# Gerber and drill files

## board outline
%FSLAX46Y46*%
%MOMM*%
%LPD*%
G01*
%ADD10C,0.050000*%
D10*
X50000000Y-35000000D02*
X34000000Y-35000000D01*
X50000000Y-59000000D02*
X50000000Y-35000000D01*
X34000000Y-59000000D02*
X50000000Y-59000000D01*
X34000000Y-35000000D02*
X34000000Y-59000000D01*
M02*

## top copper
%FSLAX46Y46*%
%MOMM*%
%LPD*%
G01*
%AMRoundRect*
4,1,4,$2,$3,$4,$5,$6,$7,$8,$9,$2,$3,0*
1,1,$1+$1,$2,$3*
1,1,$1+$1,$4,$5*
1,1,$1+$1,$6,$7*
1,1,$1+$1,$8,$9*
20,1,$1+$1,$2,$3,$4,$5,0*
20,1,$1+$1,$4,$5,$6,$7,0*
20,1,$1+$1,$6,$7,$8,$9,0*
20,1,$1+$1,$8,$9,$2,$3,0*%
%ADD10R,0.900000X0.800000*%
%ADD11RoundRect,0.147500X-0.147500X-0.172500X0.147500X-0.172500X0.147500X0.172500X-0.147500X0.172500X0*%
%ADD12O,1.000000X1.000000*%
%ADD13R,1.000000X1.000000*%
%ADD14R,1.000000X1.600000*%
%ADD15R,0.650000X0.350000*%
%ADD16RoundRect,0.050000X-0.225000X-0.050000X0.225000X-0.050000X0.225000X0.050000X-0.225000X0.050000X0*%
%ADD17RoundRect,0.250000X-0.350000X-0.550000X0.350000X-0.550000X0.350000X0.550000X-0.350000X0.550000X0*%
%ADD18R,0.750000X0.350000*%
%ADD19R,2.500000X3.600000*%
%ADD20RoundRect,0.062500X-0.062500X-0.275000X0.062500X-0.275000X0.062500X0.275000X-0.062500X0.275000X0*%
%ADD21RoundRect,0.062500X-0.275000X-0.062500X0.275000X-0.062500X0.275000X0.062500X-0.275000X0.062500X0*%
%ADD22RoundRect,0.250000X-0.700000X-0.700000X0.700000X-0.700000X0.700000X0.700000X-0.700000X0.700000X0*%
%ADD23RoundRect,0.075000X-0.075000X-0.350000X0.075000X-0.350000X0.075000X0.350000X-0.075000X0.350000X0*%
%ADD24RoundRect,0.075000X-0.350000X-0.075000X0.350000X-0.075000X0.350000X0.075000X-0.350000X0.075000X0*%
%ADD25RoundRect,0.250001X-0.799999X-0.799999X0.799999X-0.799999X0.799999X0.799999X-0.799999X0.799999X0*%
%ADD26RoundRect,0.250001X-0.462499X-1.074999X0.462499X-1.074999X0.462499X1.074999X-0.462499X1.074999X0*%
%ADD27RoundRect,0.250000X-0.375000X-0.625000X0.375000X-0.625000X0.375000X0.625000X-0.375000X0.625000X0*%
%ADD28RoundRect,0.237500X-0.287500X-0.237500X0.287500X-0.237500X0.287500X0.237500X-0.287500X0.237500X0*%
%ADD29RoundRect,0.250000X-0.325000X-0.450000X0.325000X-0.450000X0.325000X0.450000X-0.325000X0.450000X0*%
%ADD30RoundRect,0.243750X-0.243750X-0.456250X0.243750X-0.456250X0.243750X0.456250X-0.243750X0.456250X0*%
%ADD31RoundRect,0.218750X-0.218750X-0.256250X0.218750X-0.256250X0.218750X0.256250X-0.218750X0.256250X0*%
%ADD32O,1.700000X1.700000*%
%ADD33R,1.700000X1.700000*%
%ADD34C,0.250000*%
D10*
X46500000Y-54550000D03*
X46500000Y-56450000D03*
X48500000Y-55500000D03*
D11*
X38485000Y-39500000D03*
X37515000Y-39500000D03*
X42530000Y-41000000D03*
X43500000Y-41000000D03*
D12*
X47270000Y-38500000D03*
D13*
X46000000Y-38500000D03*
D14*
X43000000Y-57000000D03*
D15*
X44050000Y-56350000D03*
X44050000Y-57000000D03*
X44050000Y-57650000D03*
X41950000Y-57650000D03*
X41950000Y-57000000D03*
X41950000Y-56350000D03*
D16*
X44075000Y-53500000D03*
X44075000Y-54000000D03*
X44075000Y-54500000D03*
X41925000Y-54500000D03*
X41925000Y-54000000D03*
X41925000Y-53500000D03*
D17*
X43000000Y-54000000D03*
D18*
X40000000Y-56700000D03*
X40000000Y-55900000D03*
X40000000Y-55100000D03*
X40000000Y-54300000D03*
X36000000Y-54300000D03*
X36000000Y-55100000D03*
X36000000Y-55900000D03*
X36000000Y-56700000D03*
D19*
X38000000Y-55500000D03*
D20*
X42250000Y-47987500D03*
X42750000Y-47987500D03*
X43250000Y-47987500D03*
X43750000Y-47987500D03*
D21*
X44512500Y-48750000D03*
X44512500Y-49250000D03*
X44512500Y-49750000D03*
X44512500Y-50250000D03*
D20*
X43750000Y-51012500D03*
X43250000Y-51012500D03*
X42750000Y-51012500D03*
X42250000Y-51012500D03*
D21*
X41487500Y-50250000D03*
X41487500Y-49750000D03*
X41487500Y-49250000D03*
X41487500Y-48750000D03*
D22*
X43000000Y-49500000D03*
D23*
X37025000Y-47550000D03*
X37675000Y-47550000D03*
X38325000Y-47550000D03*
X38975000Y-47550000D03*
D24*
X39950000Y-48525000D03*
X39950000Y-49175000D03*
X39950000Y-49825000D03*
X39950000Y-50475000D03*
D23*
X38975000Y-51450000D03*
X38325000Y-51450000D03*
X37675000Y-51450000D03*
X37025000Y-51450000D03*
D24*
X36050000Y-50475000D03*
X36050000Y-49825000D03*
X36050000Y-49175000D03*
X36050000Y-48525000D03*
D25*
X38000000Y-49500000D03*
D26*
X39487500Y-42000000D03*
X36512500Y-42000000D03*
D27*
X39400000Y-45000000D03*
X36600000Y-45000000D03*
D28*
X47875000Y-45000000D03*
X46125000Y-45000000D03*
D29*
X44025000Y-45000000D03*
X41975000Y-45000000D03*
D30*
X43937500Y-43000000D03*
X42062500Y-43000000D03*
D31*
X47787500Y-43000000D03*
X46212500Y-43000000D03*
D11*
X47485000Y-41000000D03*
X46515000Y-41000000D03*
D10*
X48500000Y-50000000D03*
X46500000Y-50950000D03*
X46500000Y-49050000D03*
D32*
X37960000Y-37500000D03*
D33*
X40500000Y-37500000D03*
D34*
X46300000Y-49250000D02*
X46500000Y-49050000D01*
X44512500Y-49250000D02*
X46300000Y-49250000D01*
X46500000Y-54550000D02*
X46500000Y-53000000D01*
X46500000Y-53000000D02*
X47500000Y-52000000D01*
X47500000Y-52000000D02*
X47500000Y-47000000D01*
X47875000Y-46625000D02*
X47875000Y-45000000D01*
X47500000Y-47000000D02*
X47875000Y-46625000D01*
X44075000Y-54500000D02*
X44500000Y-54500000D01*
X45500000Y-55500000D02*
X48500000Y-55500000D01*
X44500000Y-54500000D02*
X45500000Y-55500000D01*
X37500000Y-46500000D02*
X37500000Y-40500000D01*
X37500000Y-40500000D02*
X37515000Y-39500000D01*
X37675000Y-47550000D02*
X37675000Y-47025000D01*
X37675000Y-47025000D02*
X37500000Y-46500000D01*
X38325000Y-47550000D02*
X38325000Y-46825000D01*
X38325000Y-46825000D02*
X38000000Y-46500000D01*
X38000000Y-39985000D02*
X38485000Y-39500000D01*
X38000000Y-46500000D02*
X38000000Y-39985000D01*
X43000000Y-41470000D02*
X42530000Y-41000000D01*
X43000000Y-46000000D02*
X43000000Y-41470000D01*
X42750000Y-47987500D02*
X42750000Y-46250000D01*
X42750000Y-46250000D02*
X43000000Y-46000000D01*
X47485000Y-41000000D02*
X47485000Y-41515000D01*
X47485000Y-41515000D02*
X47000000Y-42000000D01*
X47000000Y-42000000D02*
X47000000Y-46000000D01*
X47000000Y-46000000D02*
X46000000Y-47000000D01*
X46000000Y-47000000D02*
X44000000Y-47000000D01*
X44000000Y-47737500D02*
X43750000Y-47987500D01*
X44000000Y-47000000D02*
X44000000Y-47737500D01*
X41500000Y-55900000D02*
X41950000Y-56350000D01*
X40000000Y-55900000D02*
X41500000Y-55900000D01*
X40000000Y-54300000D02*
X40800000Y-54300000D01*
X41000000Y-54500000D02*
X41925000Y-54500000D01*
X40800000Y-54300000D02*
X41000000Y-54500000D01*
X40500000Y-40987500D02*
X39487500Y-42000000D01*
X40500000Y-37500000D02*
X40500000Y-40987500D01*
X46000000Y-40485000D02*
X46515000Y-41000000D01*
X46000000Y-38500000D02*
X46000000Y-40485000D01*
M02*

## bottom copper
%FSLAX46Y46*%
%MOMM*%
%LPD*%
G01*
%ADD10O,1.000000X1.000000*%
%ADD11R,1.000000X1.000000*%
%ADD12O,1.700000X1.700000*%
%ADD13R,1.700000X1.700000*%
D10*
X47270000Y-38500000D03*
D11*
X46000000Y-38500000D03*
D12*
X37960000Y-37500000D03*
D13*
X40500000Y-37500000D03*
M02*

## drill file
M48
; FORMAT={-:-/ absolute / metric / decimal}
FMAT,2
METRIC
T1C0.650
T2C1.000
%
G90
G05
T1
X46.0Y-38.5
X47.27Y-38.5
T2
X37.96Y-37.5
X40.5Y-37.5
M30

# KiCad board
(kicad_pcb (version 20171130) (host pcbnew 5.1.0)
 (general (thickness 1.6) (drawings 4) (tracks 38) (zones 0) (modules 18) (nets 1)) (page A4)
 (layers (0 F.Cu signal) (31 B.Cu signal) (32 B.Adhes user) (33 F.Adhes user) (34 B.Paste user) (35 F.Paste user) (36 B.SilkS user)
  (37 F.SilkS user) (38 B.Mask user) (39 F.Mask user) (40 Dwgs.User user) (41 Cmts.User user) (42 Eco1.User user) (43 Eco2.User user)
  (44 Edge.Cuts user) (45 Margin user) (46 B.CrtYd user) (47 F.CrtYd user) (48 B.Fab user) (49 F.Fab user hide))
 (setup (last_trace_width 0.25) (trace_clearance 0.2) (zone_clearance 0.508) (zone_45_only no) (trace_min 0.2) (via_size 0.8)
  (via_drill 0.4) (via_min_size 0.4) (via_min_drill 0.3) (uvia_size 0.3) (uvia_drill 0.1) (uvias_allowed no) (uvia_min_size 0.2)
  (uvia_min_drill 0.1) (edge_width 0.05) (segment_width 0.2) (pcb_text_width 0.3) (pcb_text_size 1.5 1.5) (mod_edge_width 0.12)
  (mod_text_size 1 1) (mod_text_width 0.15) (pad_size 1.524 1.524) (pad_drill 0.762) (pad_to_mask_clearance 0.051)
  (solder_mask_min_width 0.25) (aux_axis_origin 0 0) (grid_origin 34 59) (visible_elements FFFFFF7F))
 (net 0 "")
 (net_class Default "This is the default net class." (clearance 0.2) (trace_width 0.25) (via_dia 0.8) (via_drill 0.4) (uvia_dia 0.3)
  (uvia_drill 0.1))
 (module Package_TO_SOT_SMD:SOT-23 (layer F.Cu) (at 47.5 55.5)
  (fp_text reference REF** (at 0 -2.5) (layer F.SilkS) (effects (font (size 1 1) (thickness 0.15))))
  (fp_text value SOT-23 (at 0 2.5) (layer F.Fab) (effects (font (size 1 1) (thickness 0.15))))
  (pad 1 smd rect (at -1 -0.95) (size 0.9 0.8) (layers F.Cu F.Paste F.Mask))
  (pad 2 smd rect (at -1 0.95) (size 0.9 0.8) (layers F.Cu F.Paste F.Mask))
  (pad 3 smd rect (at 1 0) (size 0.9 0.8) (layers F.Cu F.Paste F.Mask)))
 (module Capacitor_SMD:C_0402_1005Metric (layer F.Cu) (at 38 39.5)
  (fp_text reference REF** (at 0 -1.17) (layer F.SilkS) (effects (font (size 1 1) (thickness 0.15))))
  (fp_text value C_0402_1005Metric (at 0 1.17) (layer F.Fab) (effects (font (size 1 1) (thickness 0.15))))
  (pad 2 smd roundrect (at 0.485 0) (size 0.59 0.64) (layers F.Cu F.Paste F.Mask) (roundrect_rratio 0.25))
  (pad 1 smd roundrect (at -0.485 0) (size 0.59 0.64) (layers F.Cu F.Paste F.Mask) (roundrect_rratio 0.25)))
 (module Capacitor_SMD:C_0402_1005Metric (layer F.Cu) (at 43.015 41)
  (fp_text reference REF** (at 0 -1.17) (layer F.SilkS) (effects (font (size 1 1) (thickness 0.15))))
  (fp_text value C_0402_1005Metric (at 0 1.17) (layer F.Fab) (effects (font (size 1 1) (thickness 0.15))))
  (pad 1 smd roundrect (at -0.485 0) (size 0.59 0.64) (layers F.Cu F.Paste F.Mask) (roundrect_rratio 0.25))
  (pad 2 smd roundrect (at 0.485 0) (size 0.59 0.64) (layers F.Cu F.Paste F.Mask) (roundrect_rratio 0.25)))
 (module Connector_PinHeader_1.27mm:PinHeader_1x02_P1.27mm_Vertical (layer F.Cu) (at 46 38.5 90)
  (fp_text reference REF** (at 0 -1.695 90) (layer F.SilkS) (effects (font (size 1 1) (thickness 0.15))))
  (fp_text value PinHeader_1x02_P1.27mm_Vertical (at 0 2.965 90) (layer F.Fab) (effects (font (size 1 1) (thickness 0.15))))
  (pad 2 thru_hole oval (at 0 1.27 90) (size 1 1) (drill 0.65) (layers *.Cu *.Mask))
  (pad 1 thru_hole rect (at 0 0 90) (size 1 1) (drill 0.65) (layers *.Cu *.Mask)))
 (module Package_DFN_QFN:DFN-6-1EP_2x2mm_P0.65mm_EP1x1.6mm (layer F.Cu) (at 43 57)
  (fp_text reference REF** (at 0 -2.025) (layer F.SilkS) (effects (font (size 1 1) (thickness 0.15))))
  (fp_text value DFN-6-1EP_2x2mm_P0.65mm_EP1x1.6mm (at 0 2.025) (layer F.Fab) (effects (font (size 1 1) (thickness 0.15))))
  (pad "" smd rect (at 0 0.4) (size 0.82 0.63) (layers F.Paste))
  (pad "" smd rect (at 0 -0.4) (size 0.82 0.63) (layers F.Paste)) (pad 7 smd rect (at 0 0) (size 1 1.6) (layers F.Cu F.Mask))
  (pad 6 smd rect (at 1.05 -0.65) (size 0.65 0.35) (layers F.Cu F.Paste F.Mask))
  (pad 5 smd rect (at 1.05 0) (size 0.65 0.35) (layers F.Cu F.Paste F.Mask))
  (pad 4 smd rect (at 1.05 0.65) (size 0.65 0.35) (layers F.Cu F.Paste F.Mask))
  (pad 3 smd rect (at -1.05 0.65) (size 0.65 0.35) (layers F.Cu F.Paste F.Mask))
  (pad 2 smd rect (at -1.05 0) (size 0.65 0.35) (layers F.Cu F.Paste F.Mask))
  (pad 1 smd rect (at -1.05 -0.65) (size 0.65 0.35) (layers F.Cu F.Paste F.Mask)))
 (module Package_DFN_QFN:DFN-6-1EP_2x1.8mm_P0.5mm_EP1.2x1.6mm (layer F.Cu) (at 43 54)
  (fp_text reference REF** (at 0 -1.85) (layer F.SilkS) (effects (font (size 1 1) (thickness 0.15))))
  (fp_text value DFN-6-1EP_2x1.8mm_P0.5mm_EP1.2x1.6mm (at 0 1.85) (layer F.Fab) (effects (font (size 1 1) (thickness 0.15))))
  (pad 6 smd roundrect (at 1.075 -0.5) (size 0.55 0.2) (layers F.Cu F.Paste F.Mask) (roundrect_rratio 0.25))
  (pad 5 smd roundrect (at 1.075 0) (size 0.55 0.2) (layers F.Cu F.Paste F.Mask) (roundrect_rratio 0.25))
  (pad 4 smd roundrect (at 1.075 0.5) (size 0.55 0.2) (layers F.Cu F.Paste F.Mask) (roundrect_rratio 0.25))
  (pad 3 smd roundrect (at -1.075 0.5) (size 0.55 0.2) (layers F.Cu F.Paste F.Mask) (roundrect_rratio 0.25))
  (pad 2 smd roundrect (at -1.075 0) (size 0.55 0.2) (layers F.Cu F.Paste F.Mask) (roundrect_rratio 0.25))
  (pad 1 smd roundrect (at -1.075 -0.5) (size 0.55 0.2) (layers F.Cu F.Paste F.Mask) (roundrect_rratio 0.25))
  (pad "" smd roundrect (at 0.3 0.4) (size 0.48 0.64) (layers F.Paste) (roundrect_rratio 0.25))
  (pad "" smd roundrect (at 0.3 -0.4) (size 0.48 0.64) (layers F.Paste) (roundrect_rratio 0.25))
  (pad "" smd roundrect (at -0.3 0.4) (size 0.48 0.64) (layers F.Paste) (roundrect_rratio 0.25))
  (pad "" smd roundrect (at -0.3 -0.4) (size 0.48 0.64) (layers F.Paste) (roundrect_rratio 0.25))
  (pad 7 smd roundrect (at 0 0) (size 1.2 1.6) (layers F.Cu F.Mask) (roundrect_rratio 0.208333)))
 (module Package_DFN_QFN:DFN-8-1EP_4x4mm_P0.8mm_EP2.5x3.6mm (layer F.Cu) (at 38 55.5 180)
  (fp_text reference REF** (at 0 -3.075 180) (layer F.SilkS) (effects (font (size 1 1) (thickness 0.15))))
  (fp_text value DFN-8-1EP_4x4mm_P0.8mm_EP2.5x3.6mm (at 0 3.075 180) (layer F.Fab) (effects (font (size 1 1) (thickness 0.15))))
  (pad 1 smd rect (at -2 -1.2 180) (size 0.75 0.35) (layers F.Cu F.Paste F.Mask))
  (pad 2 smd rect (at -2 -0.4 180) (size 0.75 0.35) (layers F.Cu F.Paste F.Mask))
  (pad 3 smd rect (at -2 0.4 180) (size 0.75 0.35) (layers F.Cu F.Paste F.Mask))
  (pad 4 smd rect (at -2 1.2 180) (size 0.75 0.35) (layers F.Cu F.Paste F.Mask))
  (pad 5 smd rect (at 2 1.2 180) (size 0.75 0.35) (layers F.Cu F.Paste F.Mask))
  (pad 6 smd rect (at 2 0.4 180) (size 0.75 0.35) (layers F.Cu F.Paste F.Mask))
  (pad 7 smd rect (at 2 -0.4 180) (size 0.75 0.35) (layers F.Cu F.Paste F.Mask))
  (pad 8 smd rect (at 2 -1.2 180) (size 0.75 0.35) (layers F.Cu F.Paste F.Mask))
  (pad "" smd rect (at -0.625 -1.2 180) (size 1 1) (layers F.Paste))
  (pad 9 smd rect (at 0 0 180) (size 2.5 3.6) (layers F.Cu F.Mask))
  (pad "" smd rect (at 0.625 -1.2 180) (size 1 1) (layers F.Paste))
  (pad "" smd rect (at 0.625 0 180) (size 1 1) (layers F.Paste))
  (pad "" smd rect (at -0.625 0 180) (size 1 1) (layers F.Paste))
  (pad "" smd rect (at 0.625 1.2 180) (size 1 1) (layers F.Paste))
  (pad "" smd rect (at -0.625 1.2 180) (size 1 1) (layers F.Paste)))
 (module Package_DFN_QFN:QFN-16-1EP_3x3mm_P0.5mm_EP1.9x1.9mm (layer F.Cu) (at 43 49.5)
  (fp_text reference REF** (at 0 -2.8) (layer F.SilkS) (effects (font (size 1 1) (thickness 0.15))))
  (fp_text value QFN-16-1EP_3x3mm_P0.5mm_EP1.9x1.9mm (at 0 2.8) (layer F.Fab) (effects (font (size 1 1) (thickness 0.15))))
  (pad 16 smd roundrect (at -0.75 -1.5125) (size 0.25 0.675) (layers F.Cu F.Paste F.Mask) (roundrect_rratio 0.25))
  (pad 15 smd roundrect (at -0.25 -1.5125) (size 0.25 0.675) (layers F.Cu F.Paste F.Mask) (roundrect_rratio 0.25))
  (pad 14 smd roundrect (at 0.25 -1.5125) (size 0.25 0.675) (layers F.Cu F.Paste F.Mask) (roundrect_rratio 0.25))
  (pad 13 smd roundrect (at 0.75 -1.5125) (size 0.25 0.675) (layers F.Cu F.Paste F.Mask) (roundrect_rratio 0.25))
  (pad 12 smd roundrect (at 1.5125 -0.75) (size 0.675 0.25) (layers F.Cu F.Paste F.Mask) (roundrect_rratio 0.25))
  (pad 11 smd roundrect (at 1.5125 -0.25) (size 0.675 0.25) (layers F.Cu F.Paste F.Mask) (roundrect_rratio 0.25))
  (pad 10 smd roundrect (at 1.5125 0.25) (size 0.675 0.25) (layers F.Cu F.Paste F.Mask) (roundrect_rratio 0.25))
  (pad 9 smd roundrect (at 1.5125 0.75) (size 0.675 0.25) (layers F.Cu F.Paste F.Mask) (roundrect_rratio 0.25))
  (pad 8 smd roundrect (at 0.75 1.5125) (size 0.25 0.675) (layers F.Cu F.Paste F.Mask) (roundrect_rratio 0.25))
  (pad 7 smd roundrect (at 0.25 1.5125) (size 0.25 0.675) (layers F.Cu F.Paste F.Mask) (roundrect_rratio 0.25))
  (pad 6 smd roundrect (at -0.25 1.5125) (size 0.25 0.675) (layers F.Cu F.Paste F.Mask) (roundrect_rratio 0.25))
  (pad 5 smd roundrect (at -0.75 1.5125) (size 0.25 0.675) (layers F.Cu F.Paste F.Mask) (roundrect_rratio 0.25))
  (pad 4 smd roundrect (at -1.5125 0.75) (size 0.675 0.25) (layers F.Cu F.Paste F.Mask) (roundrect_rratio 0.25))
  (pad 3 smd roundrect (at -1.5125 0.25) (size 0.675 0.25) (layers F.Cu F.Paste F.Mask) (roundrect_rratio 0.25))
  (pad 2 smd roundrect (at -1.5125 -0.25) (size 0.675 0.25) (layers F.Cu F.Paste F.Mask) (roundrect_rratio 0.25))
  (pad 1 smd roundrect (at -1.5125 -0.75) (size 0.675 0.25) (layers F.Cu F.Paste F.Mask) (roundrect_rratio 0.25))
  (pad "" smd roundrect (at 0.475 0.475) (size 0.77 0.77) (layers F.Paste) (roundrect_rratio 0.25))
  (pad "" smd roundrect (at 0.475 -0.475) (size 0.77 0.77) (layers F.Paste) (roundrect_rratio 0.25))
  (pad "" smd roundrect (at -0.475 0.475) (size 0.77 0.77) (layers F.Paste) (roundrect_rratio 0.25))
  (pad "" smd roundrect (at -0.475 -0.475) (size 0.77 0.77) (layers F.Paste) (roundrect_rratio 0.25))
  (pad 17 smd roundrect (at 0 0) (size 1.9 1.9) (layers F.Cu F.Mask) (roundrect_rratio 0.131579)))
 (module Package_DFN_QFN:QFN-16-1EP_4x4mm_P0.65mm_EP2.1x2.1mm (layer F.Cu) (at 38 49.5)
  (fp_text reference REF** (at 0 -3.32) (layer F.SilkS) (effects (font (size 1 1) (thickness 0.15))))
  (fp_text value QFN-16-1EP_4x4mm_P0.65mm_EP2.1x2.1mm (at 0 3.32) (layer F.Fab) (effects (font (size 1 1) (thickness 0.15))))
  (pad 16 smd roundrect (at -0.975 -1.95) (size 0.3 0.85) (layers F.Cu F.Paste F.Mask) (roundrect_rratio 0.25))
  (pad 15 smd roundrect (at -0.325 -1.95) (size 0.3 0.85) (layers F.Cu F.Paste F.Mask) (roundrect_rratio 0.25))
  (pad 14 smd roundrect (at 0.325 -1.95) (size 0.3 0.85) (layers F.Cu F.Paste F.Mask) (roundrect_rratio 0.25))
  (pad 13 smd roundrect (at 0.975 -1.95) (size 0.3 0.85) (layers F.Cu F.Paste F.Mask) (roundrect_rratio 0.25))
  (pad 12 smd roundrect (at 1.95 -0.975) (size 0.85 0.3) (layers F.Cu F.Paste F.Mask) (roundrect_rratio 0.25))
  (pad 11 smd roundrect (at 1.95 -0.325) (size 0.85 0.3) (layers F.Cu F.Paste F.Mask) (roundrect_rratio 0.25))
  (pad 10 smd roundrect (at 1.95 0.325) (size 0.85 0.3) (layers F.Cu F.Paste F.Mask) (roundrect_rratio 0.25))
  (pad 9 smd roundrect (at 1.95 0.975) (size 0.85 0.3) (layers F.Cu F.Paste F.Mask) (roundrect_rratio 0.25))
  (pad 8 smd roundrect (at 0.975 1.95) (size 0.3 0.85) (layers F.Cu F.Paste F.Mask) (roundrect_rratio 0.25))
  (pad 7 smd roundrect (at 0.325 1.95) (size 0.3 0.85) (layers F.Cu F.Paste F.Mask) (roundrect_rratio 0.25))
  (pad 6 smd roundrect (at -0.325 1.95) (size 0.3 0.85) (layers F.Cu F.Paste F.Mask) (roundrect_rratio 0.25))
  (pad 5 smd roundrect (at -0.975 1.95) (size 0.3 0.85) (layers F.Cu F.Paste F.Mask) (roundrect_rratio 0.25))
  (pad 4 smd roundrect (at -1.95 0.975) (size 0.85 0.3) (layers F.Cu F.Paste F.Mask) (roundrect_rratio 0.25))
  (pad 3 smd roundrect (at -1.95 0.325) (size 0.85 0.3) (layers F.Cu F.Paste F.Mask) (roundrect_rratio 0.25))
  (pad 2 smd roundrect (at -1.95 -0.325) (size 0.85 0.3) (layers F.Cu F.Paste F.Mask) (roundrect_rratio 0.25))
  (pad 1 smd roundrect (at -1.95 -0.975) (size 0.85 0.3) (layers F.Cu F.Paste F.Mask) (roundrect_rratio 0.25))
  (pad "" smd roundrect (at 0.525 0.525) (size 0.85 0.85) (layers F.Paste) (roundrect_rratio 0.25))
  (pad "" smd roundrect (at 0.525 -0.525) (size 0.85 0.85) (layers F.Paste) (roundrect_rratio 0.25))
  (pad "" smd roundrect (at -0.525 0.525) (size 0.85 0.85) (layers F.Paste) (roundrect_rratio 0.25))
  (pad "" smd roundrect (at -0.525 -0.525) (size 0.85 0.85) (layers F.Paste) (roundrect_rratio 0.25))
  (pad 17 smd roundrect (at 0 0) (size 2.1 2.1) (layers F.Cu F.Mask) (roundrect_rratio 0.119048)))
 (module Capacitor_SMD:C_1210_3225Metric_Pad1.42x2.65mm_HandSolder (layer F.Cu) (at 38 42)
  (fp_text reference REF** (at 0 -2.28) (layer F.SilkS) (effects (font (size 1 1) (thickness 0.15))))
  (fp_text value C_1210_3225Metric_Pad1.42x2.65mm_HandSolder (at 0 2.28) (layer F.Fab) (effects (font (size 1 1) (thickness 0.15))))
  (pad 2 smd roundrect (at 1.4875 0) (size 1.425 2.65) (layers F.Cu F.Paste F.Mask) (roundrect_rratio 0.175439))
  (pad 1 smd roundrect (at -1.4875 0) (size 1.425 2.65) (layers F.Cu F.Paste F.Mask) (roundrect_rratio 0.175439)))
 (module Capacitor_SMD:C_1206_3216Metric (layer F.Cu) (at 38 45)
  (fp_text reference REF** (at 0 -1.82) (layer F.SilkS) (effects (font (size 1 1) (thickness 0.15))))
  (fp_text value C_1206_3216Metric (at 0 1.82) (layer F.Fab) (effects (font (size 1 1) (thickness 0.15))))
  (pad 2 smd roundrect (at 1.4 0) (size 1.25 1.75) (layers F.Cu F.Paste F.Mask) (roundrect_rratio 0.2))
  (pad 1 smd roundrect (at -1.4 0) (size 1.25 1.75) (layers F.Cu F.Paste F.Mask) (roundrect_rratio 0.2)))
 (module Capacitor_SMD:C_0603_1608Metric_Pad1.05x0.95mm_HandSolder (layer F.Cu) (at 47 45)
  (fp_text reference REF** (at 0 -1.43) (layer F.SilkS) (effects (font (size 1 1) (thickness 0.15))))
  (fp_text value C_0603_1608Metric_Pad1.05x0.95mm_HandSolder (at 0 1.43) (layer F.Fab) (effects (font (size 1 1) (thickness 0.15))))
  (pad 2 smd roundrect (at 0.875 0) (size 1.05 0.95) (layers F.Cu F.Paste F.Mask) (roundrect_rratio 0.25))
  (pad 1 smd roundrect (at -0.875 0) (size 1.05 0.95) (layers F.Cu F.Paste F.Mask) (roundrect_rratio 0.25)))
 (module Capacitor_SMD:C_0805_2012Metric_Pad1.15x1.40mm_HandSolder (layer F.Cu) (at 43 45)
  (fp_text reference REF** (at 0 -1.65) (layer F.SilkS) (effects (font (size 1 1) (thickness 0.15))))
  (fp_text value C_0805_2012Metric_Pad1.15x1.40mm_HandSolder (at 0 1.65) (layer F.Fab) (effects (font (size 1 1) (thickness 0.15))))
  (pad 2 smd roundrect (at 1.025 0) (size 1.15 1.4) (layers F.Cu F.Paste F.Mask) (roundrect_rratio 0.217391))
  (pad 1 smd roundrect (at -1.025 0) (size 1.15 1.4) (layers F.Cu F.Paste F.Mask) (roundrect_rratio 0.217391)))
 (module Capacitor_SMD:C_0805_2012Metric (layer F.Cu) (at 43 43)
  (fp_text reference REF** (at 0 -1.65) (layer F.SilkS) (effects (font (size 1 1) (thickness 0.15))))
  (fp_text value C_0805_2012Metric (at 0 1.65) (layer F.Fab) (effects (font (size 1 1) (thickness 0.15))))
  (pad 2 smd roundrect (at 0.9375 0) (size 0.975 1.4) (layers F.Cu F.Paste F.Mask) (roundrect_rratio 0.25))
  (pad 1 smd roundrect (at -0.9375 0) (size 0.975 1.4) (layers F.Cu F.Paste F.Mask) (roundrect_rratio 0.25)))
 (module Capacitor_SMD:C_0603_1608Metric (layer F.Cu) (at 47 43)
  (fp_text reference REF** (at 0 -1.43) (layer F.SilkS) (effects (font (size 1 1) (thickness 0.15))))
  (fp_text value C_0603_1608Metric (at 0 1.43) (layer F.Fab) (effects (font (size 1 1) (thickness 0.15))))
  (pad 2 smd roundrect (at 0.7875 0) (size 0.875 0.95) (layers F.Cu F.Paste F.Mask) (roundrect_rratio 0.25))
  (pad 1 smd roundrect (at -0.7875 0) (size 0.875 0.95) (layers F.Cu F.Paste F.Mask) (roundrect_rratio 0.25)))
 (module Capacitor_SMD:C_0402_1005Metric (layer F.Cu) (at 47 41)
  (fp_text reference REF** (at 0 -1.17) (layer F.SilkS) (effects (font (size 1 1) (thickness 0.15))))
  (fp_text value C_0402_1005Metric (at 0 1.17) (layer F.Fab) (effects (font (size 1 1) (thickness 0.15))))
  (pad 2 smd roundrect (at 0.485 0) (size 0.59 0.64) (layers F.Cu F.Paste F.Mask) (roundrect_rratio 0.25))
  (pad 1 smd roundrect (at -0.485 0) (size 0.59 0.64) (layers F.Cu F.Paste F.Mask) (roundrect_rratio 0.25)))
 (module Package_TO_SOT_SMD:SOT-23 (layer F.Cu) (at 47.5 50)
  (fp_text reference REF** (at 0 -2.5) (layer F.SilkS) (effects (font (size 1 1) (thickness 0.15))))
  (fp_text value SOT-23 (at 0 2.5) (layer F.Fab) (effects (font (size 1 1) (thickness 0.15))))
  (pad 3 smd rect (at 1 0) (size 0.9 0.8) (layers F.Cu F.Paste F.Mask))
  (pad 2 smd rect (at -1 0.95) (size 0.9 0.8) (layers F.Cu F.Paste F.Mask))
  (pad 1 smd rect (at -1 -0.95) (size 0.9 0.8) (layers F.Cu F.Paste F.Mask)))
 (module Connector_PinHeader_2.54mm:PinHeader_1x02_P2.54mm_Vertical (layer F.Cu) (at 40.5 37.5 270)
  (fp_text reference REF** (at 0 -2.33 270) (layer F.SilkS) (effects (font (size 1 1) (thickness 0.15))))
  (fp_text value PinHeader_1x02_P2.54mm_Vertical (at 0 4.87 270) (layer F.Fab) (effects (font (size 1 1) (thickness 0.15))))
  (pad 2 thru_hole oval (at 0 2.54 270) (size 1.7 1.7) (drill 1) (layers *.Cu *.Mask))
  (pad 1 thru_hole rect (at 0 0 270) (size 1.7 1.7) (drill 1) (layers *.Cu *.Mask)))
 (gr_line (start 50 35) (end 34 35) (layer Edge.Cuts) (width 0.05))
 (gr_line (start 50 59) (end 50 35) (layer Edge.Cuts) (width 0.05))
 (gr_line (start 34 59) (end 50 59) (layer Edge.Cuts) (width 0.05))
 (gr_line (start 34 35) (end 34 59) (layer Edge.Cuts) (width 0.05))
 (segment (start 46.3 49.25) (end 46.5 49.05) (width 0.25) (layer F.Cu) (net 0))
 (segment (start 44.5125 49.25) (end 46.3 49.25) (width 0.25) (layer F.Cu) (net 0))
 (segment (start 46.5 54.55) (end 46.5 53) (width 0.25) (layer F.Cu) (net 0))
 (segment (start 46.5 53) (end 47.5 52) (width 0.25) (layer F.Cu) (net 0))
 (segment (start 47.5 52) (end 47.5 47) (width 0.25) (layer F.Cu) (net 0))
 (segment (start 47.875 46.625) (end 47.875 45) (width 0.25) (layer F.Cu) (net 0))
 (segment (start 47.5 47) (end 47.875 46.625) (width 0.25) (layer F.Cu) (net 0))
 (segment (start 44.075 54.5) (end 44.5 54.5) (width 0.25) (layer F.Cu) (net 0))
 (segment (start 45.5 55.5) (end 48.5 55.5) (width 0.25) (layer F.Cu) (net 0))
 (segment (start 44.5 54.5) (end 45.5 55.5) (width 0.25) (layer F.Cu) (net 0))
 (segment (start 37.5 46.5) (end 37.5 40.5) (width 0.25) (layer F.Cu) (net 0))
 (segment (start 37.5 40.5) (end 37.515 39.5) (width 0.25) (layer F.Cu) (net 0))
 (segment (start 37.675 47.55) (end 37.675 47.025) (width 0.25) (layer F.Cu) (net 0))
 (segment (start 37.675 47.025) (end 37.5 46.5) (width 0.25) (layer F.Cu) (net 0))
 (segment (start 38.325 47.55) (end 38.325 46.825) (width 0.25) (layer F.Cu) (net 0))
 (segment (start 38.325 46.825) (end 38 46.5) (width 0.25) (layer F.Cu) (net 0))
 (segment (start 38 39.985) (end 38.485 39.5) (width 0.25) (layer F.Cu) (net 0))
 (segment (start 38 46.5) (end 38 39.985) (width 0.25) (layer F.Cu) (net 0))
 (segment (start 43 41.47) (end 42.53 41) (width 0.25) (layer F.Cu) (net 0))
 (segment (start 43 46) (end 43 41.47) (width 0.25) (layer F.Cu) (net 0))
 (segment (start 42.75 47.9875) (end 42.75 46.25) (width 0.25) (layer F.Cu) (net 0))
 (segment (start 42.75 46.25) (end 43 46) (width 0.25) (layer F.Cu) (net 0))
 (segment (start 47.485 41) (end 47.485 41.515) (width 0.25) (layer F.Cu) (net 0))
 (segment (start 47.485 41.515) (end 47 42) (width 0.25) (layer F.Cu) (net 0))
 (segment (start 47 42) (end 47 46) (width 0.25) (layer F.Cu) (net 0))
 (segment (start 47 46) (end 46 47) (width 0.25) (layer F.Cu) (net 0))
 (segment (start 46 47) (end 44 47) (width 0.25) (layer F.Cu) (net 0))
 (segment (start 44 47.7375) (end 43.75 47.9875) (width 0.25) (layer F.Cu) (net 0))
 (segment (start 44 47) (end 44 47.7375) (width 0.25) (layer F.Cu) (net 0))
 (segment (start 41.5 55.9) (end 41.95 56.35) (width 0.25) (layer F.Cu) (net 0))
 (segment (start 40 55.9) (end 41.5 55.9) (width 0.25) (layer F.Cu) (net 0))
 (segment (start 40 54.3) (end 40.8 54.3) (width 0.25) (layer F.Cu) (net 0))
 (segment (start 41 54.5) (end 41.925 54.5) (width 0.25) (layer F.Cu) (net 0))
 (segment (start 40.8 54.3) (end 41 54.5) (width 0.25) (layer F.Cu) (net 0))
 (segment (start 40.5 40.9875) (end 39.4875 42) (width 0.25) (layer F.Cu) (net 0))
 (segment (start 40.5 37.5) (end 40.5 40.9875) (width 0.25) (layer F.Cu) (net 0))
 (segment (start 46 40.485) (end 46.515 41) (width 0.25) (layer F.Cu) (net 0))
 (segment (start 46 38.5) (end 46 40.485) (width 0.25) (layer F.Cu) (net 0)))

